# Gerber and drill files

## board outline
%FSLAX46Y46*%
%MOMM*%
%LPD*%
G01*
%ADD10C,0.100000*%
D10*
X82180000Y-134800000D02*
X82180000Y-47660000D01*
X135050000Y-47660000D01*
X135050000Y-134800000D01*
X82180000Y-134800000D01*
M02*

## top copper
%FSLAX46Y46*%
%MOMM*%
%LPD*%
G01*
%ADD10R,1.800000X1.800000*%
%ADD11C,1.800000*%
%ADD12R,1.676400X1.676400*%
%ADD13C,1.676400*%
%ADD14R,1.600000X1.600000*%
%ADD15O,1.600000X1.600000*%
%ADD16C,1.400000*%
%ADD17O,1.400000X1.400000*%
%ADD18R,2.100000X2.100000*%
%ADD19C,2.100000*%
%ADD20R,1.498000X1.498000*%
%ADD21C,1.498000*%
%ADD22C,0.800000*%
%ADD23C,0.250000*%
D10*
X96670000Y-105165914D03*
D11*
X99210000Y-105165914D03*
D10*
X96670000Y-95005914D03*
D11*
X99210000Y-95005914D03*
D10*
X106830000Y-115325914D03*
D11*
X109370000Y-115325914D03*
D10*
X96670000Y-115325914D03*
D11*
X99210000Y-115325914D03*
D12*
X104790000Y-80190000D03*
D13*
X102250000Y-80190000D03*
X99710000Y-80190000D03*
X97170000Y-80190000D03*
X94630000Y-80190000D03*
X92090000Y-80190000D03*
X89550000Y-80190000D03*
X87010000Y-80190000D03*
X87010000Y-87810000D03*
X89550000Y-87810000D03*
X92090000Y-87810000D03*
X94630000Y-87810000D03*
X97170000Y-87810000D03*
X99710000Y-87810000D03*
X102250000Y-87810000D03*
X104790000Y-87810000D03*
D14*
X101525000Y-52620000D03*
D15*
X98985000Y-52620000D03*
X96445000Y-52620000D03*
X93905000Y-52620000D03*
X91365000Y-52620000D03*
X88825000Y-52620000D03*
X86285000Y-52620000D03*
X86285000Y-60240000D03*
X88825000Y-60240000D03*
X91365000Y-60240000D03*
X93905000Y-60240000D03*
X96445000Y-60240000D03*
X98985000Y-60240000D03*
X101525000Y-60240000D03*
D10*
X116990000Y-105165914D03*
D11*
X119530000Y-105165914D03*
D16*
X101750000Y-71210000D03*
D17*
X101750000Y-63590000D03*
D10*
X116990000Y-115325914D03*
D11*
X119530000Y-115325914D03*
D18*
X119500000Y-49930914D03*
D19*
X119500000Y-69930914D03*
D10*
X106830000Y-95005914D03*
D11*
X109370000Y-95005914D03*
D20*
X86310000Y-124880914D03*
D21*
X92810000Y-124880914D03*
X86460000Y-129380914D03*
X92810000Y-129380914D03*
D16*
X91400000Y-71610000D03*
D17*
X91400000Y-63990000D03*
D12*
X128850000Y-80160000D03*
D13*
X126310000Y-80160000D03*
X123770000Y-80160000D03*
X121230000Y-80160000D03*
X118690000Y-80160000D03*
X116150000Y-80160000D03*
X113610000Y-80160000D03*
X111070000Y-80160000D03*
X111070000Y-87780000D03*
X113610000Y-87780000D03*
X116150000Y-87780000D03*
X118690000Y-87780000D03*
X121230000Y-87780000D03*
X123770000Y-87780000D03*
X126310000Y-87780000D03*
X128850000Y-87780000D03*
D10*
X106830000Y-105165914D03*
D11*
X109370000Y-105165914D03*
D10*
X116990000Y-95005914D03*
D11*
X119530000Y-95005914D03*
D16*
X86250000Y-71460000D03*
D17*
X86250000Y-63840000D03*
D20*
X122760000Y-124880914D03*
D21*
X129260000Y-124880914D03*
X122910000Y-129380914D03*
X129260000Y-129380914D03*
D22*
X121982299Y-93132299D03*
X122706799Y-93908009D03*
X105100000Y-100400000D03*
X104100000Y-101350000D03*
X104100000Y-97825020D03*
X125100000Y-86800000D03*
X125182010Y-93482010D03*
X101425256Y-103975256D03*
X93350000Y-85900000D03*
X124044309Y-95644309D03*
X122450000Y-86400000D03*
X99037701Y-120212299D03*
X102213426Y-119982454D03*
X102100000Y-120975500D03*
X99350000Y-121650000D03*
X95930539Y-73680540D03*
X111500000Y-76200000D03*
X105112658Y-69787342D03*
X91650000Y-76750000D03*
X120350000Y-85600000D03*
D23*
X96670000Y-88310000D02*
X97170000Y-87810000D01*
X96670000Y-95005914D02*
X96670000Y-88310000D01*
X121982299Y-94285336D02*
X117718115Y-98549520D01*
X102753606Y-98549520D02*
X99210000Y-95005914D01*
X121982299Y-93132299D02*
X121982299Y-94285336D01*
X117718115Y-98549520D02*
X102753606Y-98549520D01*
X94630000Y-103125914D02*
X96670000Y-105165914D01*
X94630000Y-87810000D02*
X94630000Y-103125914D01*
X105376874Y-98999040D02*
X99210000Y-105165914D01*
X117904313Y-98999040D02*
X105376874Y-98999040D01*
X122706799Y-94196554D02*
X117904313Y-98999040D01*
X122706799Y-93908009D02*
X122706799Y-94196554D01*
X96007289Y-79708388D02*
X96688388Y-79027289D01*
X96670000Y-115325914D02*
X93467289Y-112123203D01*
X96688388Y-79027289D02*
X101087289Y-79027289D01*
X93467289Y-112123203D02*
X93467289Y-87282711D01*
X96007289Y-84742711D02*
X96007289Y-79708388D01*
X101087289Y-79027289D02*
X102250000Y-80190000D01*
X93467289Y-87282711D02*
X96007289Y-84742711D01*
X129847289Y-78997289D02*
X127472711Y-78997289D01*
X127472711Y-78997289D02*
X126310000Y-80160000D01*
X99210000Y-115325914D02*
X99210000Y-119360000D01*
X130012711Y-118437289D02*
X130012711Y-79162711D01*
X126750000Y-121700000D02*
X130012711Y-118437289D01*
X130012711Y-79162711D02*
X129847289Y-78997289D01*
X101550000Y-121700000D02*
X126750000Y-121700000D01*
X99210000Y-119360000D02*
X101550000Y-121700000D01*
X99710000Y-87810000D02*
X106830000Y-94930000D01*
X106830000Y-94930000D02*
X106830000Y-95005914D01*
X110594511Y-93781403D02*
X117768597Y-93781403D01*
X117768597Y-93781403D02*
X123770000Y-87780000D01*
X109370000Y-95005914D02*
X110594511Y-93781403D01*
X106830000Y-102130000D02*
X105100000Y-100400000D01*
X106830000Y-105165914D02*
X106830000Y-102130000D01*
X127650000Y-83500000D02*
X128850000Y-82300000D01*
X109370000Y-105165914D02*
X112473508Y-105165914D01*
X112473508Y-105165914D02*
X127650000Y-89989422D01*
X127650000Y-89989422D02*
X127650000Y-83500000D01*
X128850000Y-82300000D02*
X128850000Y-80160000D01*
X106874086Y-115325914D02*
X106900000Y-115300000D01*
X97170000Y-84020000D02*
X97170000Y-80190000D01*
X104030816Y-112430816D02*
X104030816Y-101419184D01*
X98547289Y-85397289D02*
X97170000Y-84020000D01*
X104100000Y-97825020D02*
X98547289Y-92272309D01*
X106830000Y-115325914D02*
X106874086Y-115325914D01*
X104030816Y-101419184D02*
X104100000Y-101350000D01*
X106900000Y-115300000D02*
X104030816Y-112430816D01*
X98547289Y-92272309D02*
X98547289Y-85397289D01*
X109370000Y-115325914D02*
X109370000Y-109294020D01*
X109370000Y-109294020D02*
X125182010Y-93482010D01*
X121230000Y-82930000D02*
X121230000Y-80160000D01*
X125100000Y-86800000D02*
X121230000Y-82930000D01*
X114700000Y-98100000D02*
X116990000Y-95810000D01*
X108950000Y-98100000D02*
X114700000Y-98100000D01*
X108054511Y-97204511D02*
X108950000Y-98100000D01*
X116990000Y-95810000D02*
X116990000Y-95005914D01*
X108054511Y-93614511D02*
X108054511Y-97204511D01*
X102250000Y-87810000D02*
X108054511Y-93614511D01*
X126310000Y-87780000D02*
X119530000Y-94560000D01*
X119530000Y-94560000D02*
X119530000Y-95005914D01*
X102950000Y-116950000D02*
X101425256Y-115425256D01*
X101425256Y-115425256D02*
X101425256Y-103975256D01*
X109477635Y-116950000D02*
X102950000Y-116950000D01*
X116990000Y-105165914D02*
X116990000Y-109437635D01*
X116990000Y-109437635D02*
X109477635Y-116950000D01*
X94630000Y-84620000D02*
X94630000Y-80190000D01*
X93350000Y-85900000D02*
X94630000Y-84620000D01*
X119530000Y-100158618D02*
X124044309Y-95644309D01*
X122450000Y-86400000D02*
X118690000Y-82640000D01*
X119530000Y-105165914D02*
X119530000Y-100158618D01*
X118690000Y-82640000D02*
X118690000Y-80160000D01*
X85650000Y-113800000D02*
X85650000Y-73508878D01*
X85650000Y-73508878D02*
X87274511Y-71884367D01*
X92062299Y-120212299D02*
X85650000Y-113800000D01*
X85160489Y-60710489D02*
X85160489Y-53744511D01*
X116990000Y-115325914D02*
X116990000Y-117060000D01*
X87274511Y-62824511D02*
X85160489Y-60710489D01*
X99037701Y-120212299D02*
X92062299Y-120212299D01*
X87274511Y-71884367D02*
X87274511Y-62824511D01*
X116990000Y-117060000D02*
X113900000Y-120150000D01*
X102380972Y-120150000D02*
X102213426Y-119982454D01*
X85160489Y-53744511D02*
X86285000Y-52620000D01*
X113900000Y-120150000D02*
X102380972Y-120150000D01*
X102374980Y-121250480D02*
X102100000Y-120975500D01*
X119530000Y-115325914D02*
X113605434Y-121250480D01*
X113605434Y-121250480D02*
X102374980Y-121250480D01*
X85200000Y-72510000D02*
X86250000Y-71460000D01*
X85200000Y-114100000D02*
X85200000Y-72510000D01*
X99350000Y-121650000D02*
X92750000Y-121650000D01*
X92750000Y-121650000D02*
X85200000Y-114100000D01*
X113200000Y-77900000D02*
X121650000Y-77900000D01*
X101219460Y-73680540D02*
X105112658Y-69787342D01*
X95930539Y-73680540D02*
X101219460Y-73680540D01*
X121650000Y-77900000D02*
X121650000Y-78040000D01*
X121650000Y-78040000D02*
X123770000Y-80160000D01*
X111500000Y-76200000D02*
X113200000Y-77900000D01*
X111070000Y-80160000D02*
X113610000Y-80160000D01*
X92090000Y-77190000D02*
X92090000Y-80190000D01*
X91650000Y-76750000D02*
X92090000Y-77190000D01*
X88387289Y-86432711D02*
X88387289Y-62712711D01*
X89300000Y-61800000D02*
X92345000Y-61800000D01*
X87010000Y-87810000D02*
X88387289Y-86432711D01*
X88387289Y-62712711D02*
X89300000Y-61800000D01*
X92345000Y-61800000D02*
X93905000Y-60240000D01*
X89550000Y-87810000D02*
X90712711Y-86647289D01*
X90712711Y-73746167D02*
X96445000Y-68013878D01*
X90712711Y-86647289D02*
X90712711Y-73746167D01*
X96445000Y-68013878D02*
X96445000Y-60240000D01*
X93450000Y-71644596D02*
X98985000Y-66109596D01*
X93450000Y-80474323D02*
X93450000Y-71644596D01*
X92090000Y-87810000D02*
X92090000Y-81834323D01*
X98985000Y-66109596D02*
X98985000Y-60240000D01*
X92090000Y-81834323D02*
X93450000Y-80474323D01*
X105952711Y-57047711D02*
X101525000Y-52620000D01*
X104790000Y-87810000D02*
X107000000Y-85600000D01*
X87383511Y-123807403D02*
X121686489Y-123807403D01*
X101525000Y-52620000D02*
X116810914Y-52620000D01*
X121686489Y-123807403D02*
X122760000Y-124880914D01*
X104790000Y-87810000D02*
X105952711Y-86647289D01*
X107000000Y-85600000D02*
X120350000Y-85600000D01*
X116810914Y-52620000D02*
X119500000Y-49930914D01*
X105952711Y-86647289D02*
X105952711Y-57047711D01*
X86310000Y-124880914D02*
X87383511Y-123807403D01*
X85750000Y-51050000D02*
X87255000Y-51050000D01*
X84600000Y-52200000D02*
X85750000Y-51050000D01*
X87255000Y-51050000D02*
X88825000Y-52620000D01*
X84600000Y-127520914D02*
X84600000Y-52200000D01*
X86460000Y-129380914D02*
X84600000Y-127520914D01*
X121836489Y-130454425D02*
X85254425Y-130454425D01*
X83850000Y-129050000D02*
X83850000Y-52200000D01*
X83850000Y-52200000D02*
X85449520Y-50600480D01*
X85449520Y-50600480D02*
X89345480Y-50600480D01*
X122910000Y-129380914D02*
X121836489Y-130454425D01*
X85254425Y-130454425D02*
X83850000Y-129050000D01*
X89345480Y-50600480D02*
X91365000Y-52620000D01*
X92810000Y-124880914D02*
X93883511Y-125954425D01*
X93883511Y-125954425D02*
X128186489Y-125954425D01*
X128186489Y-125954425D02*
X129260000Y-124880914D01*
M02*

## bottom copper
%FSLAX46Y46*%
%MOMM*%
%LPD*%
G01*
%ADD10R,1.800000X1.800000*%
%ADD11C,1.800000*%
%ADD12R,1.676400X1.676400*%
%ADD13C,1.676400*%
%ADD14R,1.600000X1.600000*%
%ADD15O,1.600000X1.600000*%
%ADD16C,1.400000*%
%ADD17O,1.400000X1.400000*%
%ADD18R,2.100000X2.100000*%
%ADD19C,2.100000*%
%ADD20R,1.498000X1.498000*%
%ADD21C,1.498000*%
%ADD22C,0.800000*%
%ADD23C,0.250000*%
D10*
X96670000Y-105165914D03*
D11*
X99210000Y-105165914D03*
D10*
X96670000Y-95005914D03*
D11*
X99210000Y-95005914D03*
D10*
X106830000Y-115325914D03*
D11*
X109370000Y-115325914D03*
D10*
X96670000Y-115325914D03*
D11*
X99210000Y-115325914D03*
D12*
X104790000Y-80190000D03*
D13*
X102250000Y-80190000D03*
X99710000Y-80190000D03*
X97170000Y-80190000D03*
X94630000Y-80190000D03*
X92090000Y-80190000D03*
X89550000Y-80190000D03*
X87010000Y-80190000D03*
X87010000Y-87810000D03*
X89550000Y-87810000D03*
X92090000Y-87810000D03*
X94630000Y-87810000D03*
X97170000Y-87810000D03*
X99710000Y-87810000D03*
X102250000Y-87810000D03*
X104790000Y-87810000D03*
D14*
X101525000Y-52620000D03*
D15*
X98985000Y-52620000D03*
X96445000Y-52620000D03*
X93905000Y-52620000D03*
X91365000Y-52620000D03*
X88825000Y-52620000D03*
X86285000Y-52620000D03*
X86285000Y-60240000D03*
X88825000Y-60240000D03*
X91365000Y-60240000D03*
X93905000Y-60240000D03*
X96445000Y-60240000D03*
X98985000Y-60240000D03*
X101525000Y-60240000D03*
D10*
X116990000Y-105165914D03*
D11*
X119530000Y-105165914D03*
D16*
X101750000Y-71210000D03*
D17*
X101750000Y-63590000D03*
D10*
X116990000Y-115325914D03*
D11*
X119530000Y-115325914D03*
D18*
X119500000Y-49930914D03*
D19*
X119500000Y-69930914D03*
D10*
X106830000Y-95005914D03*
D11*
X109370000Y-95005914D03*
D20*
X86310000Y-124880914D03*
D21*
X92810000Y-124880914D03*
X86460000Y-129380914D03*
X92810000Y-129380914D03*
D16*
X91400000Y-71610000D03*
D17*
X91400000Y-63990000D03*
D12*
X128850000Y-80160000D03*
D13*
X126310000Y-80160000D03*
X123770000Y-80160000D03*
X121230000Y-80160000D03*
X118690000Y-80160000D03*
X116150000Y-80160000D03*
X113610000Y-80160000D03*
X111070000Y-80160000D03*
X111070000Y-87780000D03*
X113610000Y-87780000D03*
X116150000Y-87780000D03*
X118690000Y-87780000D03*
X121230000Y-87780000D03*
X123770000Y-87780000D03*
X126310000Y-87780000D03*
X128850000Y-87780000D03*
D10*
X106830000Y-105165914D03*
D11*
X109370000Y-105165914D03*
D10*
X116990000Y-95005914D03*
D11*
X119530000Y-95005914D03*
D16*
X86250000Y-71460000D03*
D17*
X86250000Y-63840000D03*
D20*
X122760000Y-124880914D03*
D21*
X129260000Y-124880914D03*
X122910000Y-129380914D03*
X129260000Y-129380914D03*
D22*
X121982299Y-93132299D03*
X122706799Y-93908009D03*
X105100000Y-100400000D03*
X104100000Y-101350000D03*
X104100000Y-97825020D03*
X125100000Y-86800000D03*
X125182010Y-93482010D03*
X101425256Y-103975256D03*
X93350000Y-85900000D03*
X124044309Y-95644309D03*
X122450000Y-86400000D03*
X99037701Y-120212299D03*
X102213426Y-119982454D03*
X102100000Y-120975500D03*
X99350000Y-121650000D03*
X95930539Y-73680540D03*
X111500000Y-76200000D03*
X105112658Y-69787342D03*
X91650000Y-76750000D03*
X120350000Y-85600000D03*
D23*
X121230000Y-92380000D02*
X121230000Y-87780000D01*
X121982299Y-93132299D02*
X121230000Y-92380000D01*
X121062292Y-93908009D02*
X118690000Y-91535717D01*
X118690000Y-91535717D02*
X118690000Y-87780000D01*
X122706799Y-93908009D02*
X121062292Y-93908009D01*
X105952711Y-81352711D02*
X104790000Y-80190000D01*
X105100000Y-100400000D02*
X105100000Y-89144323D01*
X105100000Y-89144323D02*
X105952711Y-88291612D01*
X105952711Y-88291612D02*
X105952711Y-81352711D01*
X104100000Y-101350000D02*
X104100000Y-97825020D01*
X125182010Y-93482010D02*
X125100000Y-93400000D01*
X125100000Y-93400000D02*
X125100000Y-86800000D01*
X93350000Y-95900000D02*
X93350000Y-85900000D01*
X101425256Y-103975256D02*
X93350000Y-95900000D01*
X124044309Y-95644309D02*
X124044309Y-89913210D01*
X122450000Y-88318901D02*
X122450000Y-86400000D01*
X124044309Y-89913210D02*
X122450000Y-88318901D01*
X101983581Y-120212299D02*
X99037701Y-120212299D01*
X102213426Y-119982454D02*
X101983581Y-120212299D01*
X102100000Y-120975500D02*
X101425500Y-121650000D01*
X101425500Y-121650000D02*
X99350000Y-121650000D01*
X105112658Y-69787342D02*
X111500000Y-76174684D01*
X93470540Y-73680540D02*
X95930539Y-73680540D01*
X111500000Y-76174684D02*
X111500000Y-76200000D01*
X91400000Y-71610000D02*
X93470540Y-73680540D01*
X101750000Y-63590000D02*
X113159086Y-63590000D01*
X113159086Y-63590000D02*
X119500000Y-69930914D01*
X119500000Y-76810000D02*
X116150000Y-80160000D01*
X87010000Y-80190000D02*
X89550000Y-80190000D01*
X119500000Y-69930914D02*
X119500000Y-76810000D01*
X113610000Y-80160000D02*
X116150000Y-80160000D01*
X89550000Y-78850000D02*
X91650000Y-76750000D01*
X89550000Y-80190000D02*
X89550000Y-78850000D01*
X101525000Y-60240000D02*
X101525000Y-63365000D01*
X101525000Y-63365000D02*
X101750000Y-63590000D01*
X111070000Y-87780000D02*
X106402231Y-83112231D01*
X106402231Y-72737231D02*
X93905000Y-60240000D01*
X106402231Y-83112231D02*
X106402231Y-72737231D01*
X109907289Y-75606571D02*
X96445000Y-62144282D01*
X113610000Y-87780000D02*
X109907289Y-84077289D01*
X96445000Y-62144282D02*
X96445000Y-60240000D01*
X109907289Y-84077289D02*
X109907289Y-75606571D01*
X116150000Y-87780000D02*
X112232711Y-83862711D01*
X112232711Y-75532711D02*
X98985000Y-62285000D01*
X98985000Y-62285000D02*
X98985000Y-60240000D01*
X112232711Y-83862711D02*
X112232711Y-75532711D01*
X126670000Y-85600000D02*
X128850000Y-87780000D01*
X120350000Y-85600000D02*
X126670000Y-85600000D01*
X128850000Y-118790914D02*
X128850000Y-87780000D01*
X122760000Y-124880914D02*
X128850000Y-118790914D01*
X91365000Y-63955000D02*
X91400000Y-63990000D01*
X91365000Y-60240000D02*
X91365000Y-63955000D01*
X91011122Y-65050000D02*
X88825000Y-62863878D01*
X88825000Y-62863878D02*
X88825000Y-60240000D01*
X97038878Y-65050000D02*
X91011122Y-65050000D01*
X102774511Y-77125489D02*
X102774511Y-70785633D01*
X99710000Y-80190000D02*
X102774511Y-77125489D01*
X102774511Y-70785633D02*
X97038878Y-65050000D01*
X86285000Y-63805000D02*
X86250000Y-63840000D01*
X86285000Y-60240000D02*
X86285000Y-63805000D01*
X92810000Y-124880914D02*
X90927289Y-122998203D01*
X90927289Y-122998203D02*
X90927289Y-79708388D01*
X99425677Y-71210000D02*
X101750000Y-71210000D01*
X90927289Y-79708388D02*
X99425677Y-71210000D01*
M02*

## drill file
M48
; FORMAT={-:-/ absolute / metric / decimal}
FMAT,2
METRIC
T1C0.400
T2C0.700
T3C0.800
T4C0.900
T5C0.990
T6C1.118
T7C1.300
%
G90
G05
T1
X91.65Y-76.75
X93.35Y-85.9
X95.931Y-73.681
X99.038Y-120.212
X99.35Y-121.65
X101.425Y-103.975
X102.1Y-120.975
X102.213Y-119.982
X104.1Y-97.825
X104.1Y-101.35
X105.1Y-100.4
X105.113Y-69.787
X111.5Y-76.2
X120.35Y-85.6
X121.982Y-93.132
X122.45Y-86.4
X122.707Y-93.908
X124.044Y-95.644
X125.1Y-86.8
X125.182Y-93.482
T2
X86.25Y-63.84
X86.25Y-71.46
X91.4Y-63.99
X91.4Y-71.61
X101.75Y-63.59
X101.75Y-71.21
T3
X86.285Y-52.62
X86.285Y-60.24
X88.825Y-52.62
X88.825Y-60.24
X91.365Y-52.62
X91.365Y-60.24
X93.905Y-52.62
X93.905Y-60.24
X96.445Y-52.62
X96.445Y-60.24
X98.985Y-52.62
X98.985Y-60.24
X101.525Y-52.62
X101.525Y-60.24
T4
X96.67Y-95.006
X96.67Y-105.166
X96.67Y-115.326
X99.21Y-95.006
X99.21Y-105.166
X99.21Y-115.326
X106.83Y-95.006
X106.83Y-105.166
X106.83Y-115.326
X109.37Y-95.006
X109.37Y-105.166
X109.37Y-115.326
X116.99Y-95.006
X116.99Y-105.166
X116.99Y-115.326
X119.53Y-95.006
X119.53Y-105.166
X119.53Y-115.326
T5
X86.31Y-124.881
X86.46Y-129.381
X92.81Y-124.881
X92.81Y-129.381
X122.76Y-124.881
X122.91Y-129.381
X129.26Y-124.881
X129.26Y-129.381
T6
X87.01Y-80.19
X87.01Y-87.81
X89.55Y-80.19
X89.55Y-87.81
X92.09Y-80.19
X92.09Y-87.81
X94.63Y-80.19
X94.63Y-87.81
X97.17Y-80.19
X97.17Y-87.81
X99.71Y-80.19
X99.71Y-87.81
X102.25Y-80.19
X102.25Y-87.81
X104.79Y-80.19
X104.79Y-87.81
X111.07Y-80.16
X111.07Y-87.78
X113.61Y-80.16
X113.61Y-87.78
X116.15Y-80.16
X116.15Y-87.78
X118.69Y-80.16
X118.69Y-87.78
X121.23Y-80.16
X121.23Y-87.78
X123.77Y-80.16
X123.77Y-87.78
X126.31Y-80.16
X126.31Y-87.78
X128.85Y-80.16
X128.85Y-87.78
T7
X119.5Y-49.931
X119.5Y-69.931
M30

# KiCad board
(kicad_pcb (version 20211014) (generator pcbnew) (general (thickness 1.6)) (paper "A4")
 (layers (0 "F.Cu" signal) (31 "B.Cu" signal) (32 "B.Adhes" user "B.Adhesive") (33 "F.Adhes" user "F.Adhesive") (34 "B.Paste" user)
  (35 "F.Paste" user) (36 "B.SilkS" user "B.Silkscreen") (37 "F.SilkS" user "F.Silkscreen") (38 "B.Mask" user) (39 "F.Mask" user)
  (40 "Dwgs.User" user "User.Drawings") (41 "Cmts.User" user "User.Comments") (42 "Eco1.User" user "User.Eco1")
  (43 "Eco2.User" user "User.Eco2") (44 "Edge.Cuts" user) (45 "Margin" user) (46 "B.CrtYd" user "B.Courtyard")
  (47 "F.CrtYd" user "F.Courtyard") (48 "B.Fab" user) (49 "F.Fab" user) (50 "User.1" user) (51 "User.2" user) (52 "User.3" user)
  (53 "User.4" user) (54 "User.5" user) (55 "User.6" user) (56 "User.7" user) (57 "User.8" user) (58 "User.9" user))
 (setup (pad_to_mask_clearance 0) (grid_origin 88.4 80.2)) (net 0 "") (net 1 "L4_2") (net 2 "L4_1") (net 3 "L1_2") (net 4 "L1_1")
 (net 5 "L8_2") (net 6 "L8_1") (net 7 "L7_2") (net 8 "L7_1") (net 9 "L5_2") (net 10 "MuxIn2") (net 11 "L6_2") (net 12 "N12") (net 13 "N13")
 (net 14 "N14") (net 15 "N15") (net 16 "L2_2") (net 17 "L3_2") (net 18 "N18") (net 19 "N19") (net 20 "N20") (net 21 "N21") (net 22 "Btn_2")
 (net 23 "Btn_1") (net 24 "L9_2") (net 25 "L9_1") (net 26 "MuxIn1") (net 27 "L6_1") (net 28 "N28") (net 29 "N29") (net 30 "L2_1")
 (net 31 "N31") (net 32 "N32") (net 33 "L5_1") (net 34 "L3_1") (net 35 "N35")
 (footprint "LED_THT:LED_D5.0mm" (layer "F.Cu") (at 96.67 105.165914)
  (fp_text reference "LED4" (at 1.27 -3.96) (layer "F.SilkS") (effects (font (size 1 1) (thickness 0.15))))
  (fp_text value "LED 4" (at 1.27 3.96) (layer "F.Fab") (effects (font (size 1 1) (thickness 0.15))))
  (pad "1" thru_hole rect (at 0 0) (size 1.8 1.8) (drill 0.9) (layers *.Cu *.Mask) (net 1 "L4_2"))
  (pad "2" thru_hole circle (at 2.54 0) (size 1.8 1.8) (drill 0.9) (layers *.Cu *.Mask) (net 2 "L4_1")))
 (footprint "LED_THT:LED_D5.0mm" (layer "F.Cu") (at 96.67 95.005914)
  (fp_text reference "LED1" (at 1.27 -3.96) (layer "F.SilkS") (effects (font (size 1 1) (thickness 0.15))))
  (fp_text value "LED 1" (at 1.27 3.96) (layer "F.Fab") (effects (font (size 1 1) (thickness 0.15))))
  (pad "1" thru_hole rect (at 0 0) (size 1.8 1.8) (drill 0.9) (layers *.Cu *.Mask) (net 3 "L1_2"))
  (pad "2" thru_hole circle (at 2.54 0) (size 1.8 1.8) (drill 0.9) (layers *.Cu *.Mask) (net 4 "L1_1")))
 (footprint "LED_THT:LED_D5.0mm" (layer "F.Cu") (at 106.83 115.325914)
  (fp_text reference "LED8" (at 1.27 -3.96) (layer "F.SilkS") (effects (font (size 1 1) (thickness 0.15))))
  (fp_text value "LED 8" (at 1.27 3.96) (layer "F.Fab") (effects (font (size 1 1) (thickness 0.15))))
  (pad "1" thru_hole rect (at 0 0) (size 1.8 1.8) (drill 0.9) (layers *.Cu *.Mask) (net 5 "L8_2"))
  (pad "2" thru_hole circle (at 2.54 0) (size 1.8 1.8) (drill 0.9) (layers *.Cu *.Mask) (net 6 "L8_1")))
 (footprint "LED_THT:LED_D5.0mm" (layer "F.Cu") (at 96.67 115.325914)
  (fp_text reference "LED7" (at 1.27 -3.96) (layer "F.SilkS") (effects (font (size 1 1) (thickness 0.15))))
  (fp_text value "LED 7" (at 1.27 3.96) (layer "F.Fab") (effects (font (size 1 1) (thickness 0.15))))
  (pad "1" thru_hole rect (at 0 0) (size 1.8 1.8) (drill 0.9) (layers *.Cu *.Mask) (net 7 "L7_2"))
  (pad "2" thru_hole circle (at 2.54 0) (size 1.8 1.8) (drill 0.9) (layers *.Cu *.Mask) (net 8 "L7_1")))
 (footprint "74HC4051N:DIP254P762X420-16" (layer "F.Cu") (at 87.01 87.81 -90)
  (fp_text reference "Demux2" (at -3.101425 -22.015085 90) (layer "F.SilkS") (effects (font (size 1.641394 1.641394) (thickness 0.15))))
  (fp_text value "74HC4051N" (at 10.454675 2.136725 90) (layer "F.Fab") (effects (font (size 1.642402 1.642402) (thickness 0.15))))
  (pad "1" thru_hole rect locked (at -7.62 -17.78 270) (size 1.6764 1.6764) (drill 1.1176) (layers *.Cu *.Mask) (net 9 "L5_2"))
  (pad "2" thru_hole circle locked (at -7.62 -15.24 270) (size 1.6764 1.6764) (drill 1.1176) (layers *.Cu *.Mask) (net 7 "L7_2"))
  (pad "3" thru_hole circle locked (at -7.62 -12.7 270) (size 1.6764 1.6764) (drill 1.1176) (layers *.Cu *.Mask) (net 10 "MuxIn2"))
  (pad "4" thru_hole circle locked (at -7.62 -10.16 270) (size 1.6764 1.6764) (drill 1.1176) (layers *.Cu *.Mask) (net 5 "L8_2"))
  (pad "5" thru_hole circle locked (at -7.62 -7.62 270) (size 1.6764 1.6764) (drill 1.1176) (layers *.Cu *.Mask) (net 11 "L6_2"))
  (pad "6" thru_hole circle locked (at -7.62 -5.08 270) (size 1.6764 1.6764) (drill 1.1176) (layers *.Cu *.Mask) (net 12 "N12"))
  (pad "7" thru_hole circle locked (at -7.62 -2.54 270) (size 1.6764 1.6764) (drill 1.1176) (layers *.Cu *.Mask) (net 12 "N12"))
  (pad "8" thru_hole circle locked (at -7.62 0 270) (size 1.6764 1.6764) (drill 1.1176) (layers *.Cu *.Mask) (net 12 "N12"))
  (pad "9" thru_hole circle locked (at 0 0 270) (size 1.6764 1.6764) (drill 1.1176) (layers *.Cu *.Mask) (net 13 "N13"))
  (pad "10" thru_hole circle locked (at 0 -2.54 270) (size 1.6764 1.6764) (drill 1.1176) (layers *.Cu *.Mask) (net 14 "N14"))
  (pad "11" thru_hole circle locked (at 0 -5.08 270) (size 1.6764 1.6764) (drill 1.1176) (layers *.Cu *.Mask) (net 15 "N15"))
  (pad "12" thru_hole circle locked (at 0 -7.62 270) (size 1.6764 1.6764) (drill 1.1176) (layers *.Cu *.Mask) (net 1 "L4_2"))
  (pad "13" thru_hole circle locked (at 0 -10.16 270) (size 1.6764 1.6764) (drill 1.1176) (layers *.Cu *.Mask) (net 3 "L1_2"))
  (pad "14" thru_hole circle locked (at 0 -12.7 270) (size 1.6764 1.6764) (drill 1.1176) (layers *.Cu *.Mask) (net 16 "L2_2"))
  (pad "15" thru_hole circle locked (at 0 -15.24 270) (size 1.6764 1.6764) (drill 1.1176) (layers *.Cu *.Mask) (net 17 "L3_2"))
  (pad "16" thru_hole circle locked (at 0 -17.78 270) (size 1.6764 1.6764) (drill 1.1176) (layers *.Cu *.Mask) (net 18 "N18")))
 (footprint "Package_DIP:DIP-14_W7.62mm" (layer "F.Cu") (at 101.525 52.62 -90)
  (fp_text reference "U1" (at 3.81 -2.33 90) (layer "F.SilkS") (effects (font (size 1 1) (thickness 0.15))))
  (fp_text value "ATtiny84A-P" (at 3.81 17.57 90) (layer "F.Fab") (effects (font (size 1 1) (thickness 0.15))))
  (pad "1" thru_hole rect (at 0 0 270) (size 1.6 1.6) (drill 0.8) (layers *.Cu *.Mask) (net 18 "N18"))
  (pad "2" thru_hole oval (at 0 2.54 270) (size 1.6 1.6) (drill 0.8) (layers *.Cu *.Mask) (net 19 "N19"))
  (pad "3" thru_hole oval (at 0 5.08 270) (size 1.6 1.6) (drill 0.8) (layers *.Cu *.Mask) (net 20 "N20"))
  (pad "4" thru_hole oval (at 0 7.62 270) (size 1.6 1.6) (drill 0.8) (layers *.Cu *.Mask) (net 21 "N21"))
  (pad "5" thru_hole oval (at 0 10.16 270) (size 1.6 1.6) (drill 0.8) (layers *.Cu *.Mask) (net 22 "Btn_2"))
  (pad "6" thru_hole oval (at 0 12.7 270) (size 1.6 1.6) (drill 0.8) (layers *.Cu *.Mask) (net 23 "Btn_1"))
  (pad "7" thru_hole oval (at 0 15.24 270) (size 1.6 1.6) (drill 0.8) (layers *.Cu *.Mask) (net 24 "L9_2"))
  (pad "8" thru_hole oval (at 7.62 15.24 270) (size 1.6 1.6) (drill 0.8) (layers *.Cu *.Mask) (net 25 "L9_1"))
  (pad "9" thru_hole oval (at 7.62 12.7 270) (size 1.6 1.6) (drill 0.8) (layers *.Cu *.Mask) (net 10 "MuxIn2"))
  (pad "10" thru_hole oval (at 7.62 10.16 270) (size 1.6 1.6) (drill 0.8) (layers *.Cu *.Mask) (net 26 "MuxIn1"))
  (pad "11" thru_hole oval (at 7.62 7.62 270) (size 1.6 1.6) (drill 0.8) (layers *.Cu *.Mask) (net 13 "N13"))
  (pad "12" thru_hole oval (at 7.62 5.08 270) (size 1.6 1.6) (drill 0.8) (layers *.Cu *.Mask) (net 14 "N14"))
  (pad "13" thru_hole oval (at 7.62 2.54 270) (size 1.6 1.6) (drill 0.8) (layers *.Cu *.Mask) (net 15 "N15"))
  (pad "14" thru_hole oval (at 7.62 0 270) (size 1.6 1.6) (drill 0.8) (layers *.Cu *.Mask) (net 12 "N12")))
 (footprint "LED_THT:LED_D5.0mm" (layer "F.Cu") (at 116.99 105.165914)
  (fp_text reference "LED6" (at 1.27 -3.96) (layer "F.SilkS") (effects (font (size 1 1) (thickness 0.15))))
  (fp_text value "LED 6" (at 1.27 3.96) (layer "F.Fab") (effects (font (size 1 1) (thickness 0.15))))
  (pad "1" thru_hole rect (at 0 0) (size 1.8 1.8) (drill 0.9) (layers *.Cu *.Mask) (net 11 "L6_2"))
  (pad "2" thru_hole circle (at 2.54 0) (size 1.8 1.8) (drill 0.9) (layers *.Cu *.Mask) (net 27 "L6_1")))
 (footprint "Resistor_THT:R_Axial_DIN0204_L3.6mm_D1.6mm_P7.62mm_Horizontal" (layer "F.Cu") (at 101.75 71.21 90)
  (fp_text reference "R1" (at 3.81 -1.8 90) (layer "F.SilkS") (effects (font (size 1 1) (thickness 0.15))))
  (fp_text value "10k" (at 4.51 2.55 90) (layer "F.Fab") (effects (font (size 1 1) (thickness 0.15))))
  (pad "1" thru_hole circle (at 0 0 90) (size 1.4 1.4) (drill 0.7) (layers *.Cu *.Mask) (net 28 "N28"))
  (pad "2" thru_hole oval (at 7.62 0 90) (size 1.4 1.4) (drill 0.7) (layers *.Cu *.Mask) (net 12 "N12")))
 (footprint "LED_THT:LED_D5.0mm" (layer "F.Cu") (at 116.99 115.325914)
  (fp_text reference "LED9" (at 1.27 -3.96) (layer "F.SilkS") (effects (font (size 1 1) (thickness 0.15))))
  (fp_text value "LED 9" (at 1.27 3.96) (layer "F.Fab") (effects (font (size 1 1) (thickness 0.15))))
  (pad "1" thru_hole rect (at 0 0) (size 1.8 1.8) (drill 0.9) (layers *.Cu *.Mask) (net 24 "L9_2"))
  (pad "2" thru_hole circle (at 2.54 0) (size 1.8 1.8) (drill 0.9) (layers *.Cu *.Mask) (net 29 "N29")))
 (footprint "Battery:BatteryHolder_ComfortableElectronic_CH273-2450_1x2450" (layer "F.Cu") (at 119.5 49.930914 -90)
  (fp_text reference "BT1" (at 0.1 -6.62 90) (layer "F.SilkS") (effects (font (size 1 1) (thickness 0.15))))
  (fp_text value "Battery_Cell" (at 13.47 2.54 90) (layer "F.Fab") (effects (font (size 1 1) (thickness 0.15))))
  (pad "1" thru_hole rect (at 0 0 180) (size 2.1 2.1) (drill 1.3) (layers *.Cu *.Mask) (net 18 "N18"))
  (pad "2" thru_hole circle (at 20 0 180) (size 2.1 2.1) (drill 1.3) (layers *.Cu *.Mask) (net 12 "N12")))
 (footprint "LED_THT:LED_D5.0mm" (layer "F.Cu") (at 106.83 95.005914)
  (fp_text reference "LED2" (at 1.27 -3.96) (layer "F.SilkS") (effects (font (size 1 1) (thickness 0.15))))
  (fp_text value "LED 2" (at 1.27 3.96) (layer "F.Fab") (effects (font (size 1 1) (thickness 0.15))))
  (pad "1" thru_hole rect (at 0 0) (size 1.8 1.8) (drill 0.9) (layers *.Cu *.Mask) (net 16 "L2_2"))
  (pad "2" thru_hole circle (at 2.54 0) (size 1.8 1.8) (drill 0.9) (layers *.Cu *.Mask) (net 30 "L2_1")))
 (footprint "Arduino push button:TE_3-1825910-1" (layer "F.Cu") (at 89.56 127.130914)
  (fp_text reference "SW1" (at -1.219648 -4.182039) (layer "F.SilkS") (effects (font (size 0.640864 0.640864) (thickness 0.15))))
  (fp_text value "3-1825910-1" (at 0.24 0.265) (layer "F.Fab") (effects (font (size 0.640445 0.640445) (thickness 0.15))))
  (pad "1" thru_hole rect locked (at -3.25 -2.25) (size 1.498 1.498) (drill 0.99) (layers *.Cu *.Mask) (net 18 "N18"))
  (pad "2" thru_hole circle locked (at 3.25 -2.25) (size 1.498 1.498) (drill 0.99) (layers *.Cu *.Mask) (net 28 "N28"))
  (pad "3" thru_hole circle locked (at -3.1 2.25) (size 1.498 1.498) (drill 0.99) (layers *.Cu *.Mask) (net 23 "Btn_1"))
  (pad "4" thru_hole circle locked (at 3.25 2.25) (size 1.498 1.498) (drill 0.99) (layers *.Cu *.Mask) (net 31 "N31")))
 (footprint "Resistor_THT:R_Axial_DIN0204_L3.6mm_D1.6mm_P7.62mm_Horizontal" (layer "F.Cu") (at 91.4 71.61 90)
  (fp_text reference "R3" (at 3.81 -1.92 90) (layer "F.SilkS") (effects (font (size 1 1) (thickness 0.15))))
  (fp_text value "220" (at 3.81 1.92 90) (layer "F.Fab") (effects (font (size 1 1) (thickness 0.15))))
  (pad "1" thru_hole circle (at 0 0 90) (size 1.4 1.4) (drill 0.7) (layers *.Cu *.Mask) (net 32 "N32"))
  (pad "2" thru_hole oval (at 7.62 0 90) (size 1.4 1.4) (drill 0.7) (layers *.Cu *.Mask) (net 26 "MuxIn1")))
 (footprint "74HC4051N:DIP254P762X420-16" (layer "F.Cu") (at 111.07 87.78 -90)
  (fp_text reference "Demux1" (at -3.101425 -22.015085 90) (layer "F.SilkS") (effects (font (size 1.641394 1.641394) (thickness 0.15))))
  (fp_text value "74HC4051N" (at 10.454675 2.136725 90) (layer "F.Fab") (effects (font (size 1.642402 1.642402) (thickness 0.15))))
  (pad "1" thru_hole rect locked (at -7.62 -17.78 270) (size 1.6764 1.6764) (drill 1.1176) (layers *.Cu *.Mask) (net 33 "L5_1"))
  (pad "2" thru_hole circle locked (at -7.62 -15.24 270) (size 1.6764 1.6764) (drill 1.1176) (layers *.Cu *.Mask) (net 8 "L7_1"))
  (pad "3" thru_hole circle locked (at -7.62 -12.7 270) (size 1.6764 1.6764) (drill 1.1176) (layers *.Cu *.Mask) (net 32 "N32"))
  (pad "4" thru_hole circle locked (at -7.62 -10.16 270) (size 1.6764 1.6764) (drill 1.1176) (layers *.Cu *.Mask) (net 6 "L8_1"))
  (pad "5" thru_hole circle locked (at -7.62 -7.62 270) (size 1.6764 1.6764) (drill 1.1176) (layers *.Cu *.Mask) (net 27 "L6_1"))
  (pad "6" thru_hole circle locked (at -7.62 -5.08 270) (size 1.6764 1.6764) (drill 1.1176) (layers *.Cu *.Mask) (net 12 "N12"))
  (pad "7" thru_hole circle locked (at -7.62 -2.54 270) (size 1.6764 1.6764) (drill 1.1176) (layers *.Cu *.Mask) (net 12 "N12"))
  (pad "8" thru_hole circle locked (at -7.62 0 270) (size 1.6764 1.6764) (drill 1.1176) (layers *.Cu *.Mask) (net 12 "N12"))
  (pad "9" thru_hole circle locked (at 0 0 270) (size 1.6764 1.6764) (drill 1.1176) (layers *.Cu *.Mask) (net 13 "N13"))
  (pad "10" thru_hole circle locked (at 0 -2.54 270) (size 1.6764 1.6764) (drill 1.1176) (layers *.Cu *.Mask) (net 14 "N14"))
  (pad "11" thru_hole circle locked (at 0 -5.08 270) (size 1.6764 1.6764) (drill 1.1176) (layers *.Cu *.Mask) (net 15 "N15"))
  (pad "12" thru_hole circle locked (at 0 -7.62 270) (size 1.6764 1.6764) (drill 1.1176) (layers *.Cu *.Mask) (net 2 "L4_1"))
  (pad "13" thru_hole circle locked (at 0 -10.16 270) (size 1.6764 1.6764) (drill 1.1176) (layers *.Cu *.Mask) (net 4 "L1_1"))
  (pad "14" thru_hole circle locked (at 0 -12.7 270) (size 1.6764 1.6764) (drill 1.1176) (layers *.Cu *.Mask) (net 30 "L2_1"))
  (pad "15" thru_hole circle locked (at 0 -15.24 270) (size 1.6764 1.6764) (drill 1.1176) (layers *.Cu *.Mask) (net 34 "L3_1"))
  (pad "16" thru_hole circle locked (at 0 -17.78 270) (size 1.6764 1.6764) (drill 1.1176) (layers *.Cu *.Mask) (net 18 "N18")))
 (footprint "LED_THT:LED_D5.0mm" (layer "F.Cu") (at 106.83 105.165914)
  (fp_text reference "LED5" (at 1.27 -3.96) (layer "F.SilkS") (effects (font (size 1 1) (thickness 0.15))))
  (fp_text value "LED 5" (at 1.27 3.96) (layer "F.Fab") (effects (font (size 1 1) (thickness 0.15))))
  (pad "1" thru_hole rect (at 0 0) (size 1.8 1.8) (drill 0.9) (layers *.Cu *.Mask) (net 9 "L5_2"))
  (pad "2" thru_hole circle (at 2.54 0) (size 1.8 1.8) (drill 0.9) (layers *.Cu *.Mask) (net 33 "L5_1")))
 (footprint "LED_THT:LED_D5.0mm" (layer "F.Cu") (at 116.99 95.005914)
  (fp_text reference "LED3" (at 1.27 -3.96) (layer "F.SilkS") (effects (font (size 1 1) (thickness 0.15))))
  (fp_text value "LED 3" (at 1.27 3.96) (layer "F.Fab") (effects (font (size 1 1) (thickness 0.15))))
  (pad "1" thru_hole rect (at 0 0) (size 1.8 1.8) (drill 0.9) (layers *.Cu *.Mask) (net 17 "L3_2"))
  (pad "2" thru_hole circle (at 2.54 0) (size 1.8 1.8) (drill 0.9) (layers *.Cu *.Mask) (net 34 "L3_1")))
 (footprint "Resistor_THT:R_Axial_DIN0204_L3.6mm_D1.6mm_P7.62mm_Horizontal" (layer "F.Cu") (at 86.25 71.46 90)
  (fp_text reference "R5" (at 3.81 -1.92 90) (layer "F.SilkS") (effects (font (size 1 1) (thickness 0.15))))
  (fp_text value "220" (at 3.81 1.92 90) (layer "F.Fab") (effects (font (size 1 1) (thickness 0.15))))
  (pad "1" thru_hole circle (at 0 0 90) (size 1.4 1.4) (drill 0.7) (layers *.Cu *.Mask) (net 29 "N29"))
  (pad "2" thru_hole oval (at 7.62 0 90) (size 1.4 1.4) (drill 0.7) (layers *.Cu *.Mask) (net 25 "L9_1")))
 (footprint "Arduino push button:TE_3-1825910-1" (layer "F.Cu") (at 126.01 127.130914)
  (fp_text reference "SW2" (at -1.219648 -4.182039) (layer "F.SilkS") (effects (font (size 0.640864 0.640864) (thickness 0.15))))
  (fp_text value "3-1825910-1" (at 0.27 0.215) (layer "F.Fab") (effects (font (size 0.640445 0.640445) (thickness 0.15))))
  (pad "1" thru_hole rect locked (at -3.25 -2.25) (size 1.498 1.498) (drill 0.99) (layers *.Cu *.Mask) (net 18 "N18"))
  (pad "2" thru_hole circle locked (at 3.25 -2.25) (size 1.498 1.498) (drill 0.99) (layers *.Cu *.Mask) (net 28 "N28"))
  (pad "3" thru_hole circle locked (at -3.1 2.25) (size 1.498 1.498) (drill 0.99) (layers *.Cu *.Mask) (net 22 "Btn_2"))
  (pad "4" thru_hole circle locked (at 3.25 2.25) (size 1.498 1.498) (drill 0.99) (layers *.Cu *.Mask) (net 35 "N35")))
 (gr_poly (pts (xy 82.18 134.8) (xy 82.18 47.66) (xy 135.05 47.66) (xy 135.05 134.8)) (layer "Edge.Cuts") (width 0.1) (fill none))
 (segment (start 96.67 88.31) (end 97.17 87.81) (width 0.25) (layer "F.Cu") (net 3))
 (segment (start 96.67 95.005914) (end 96.67 88.31) (width 0.25) (layer "F.Cu") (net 3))
 (segment (start 121.982299 94.285336) (end 117.718115 98.54952) (width 0.25) (layer "F.Cu") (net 4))
 (segment (start 102.753606 98.54952) (end 99.21 95.005914) (width 0.25) (layer "F.Cu") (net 4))
 (segment (start 121.982299 93.132299) (end 121.982299 94.285336) (width 0.25) (layer "F.Cu") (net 4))
 (segment (start 117.718115 98.54952) (end 102.753606 98.54952) (width 0.25) (layer "F.Cu") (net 4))
 (via (at 121.982299 93.132299) (size 0.8) (drill 0.4) (layers "F.Cu" "B.Cu") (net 4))
 (segment (start 121.23 92.38) (end 121.23 87.78) (width 0.25) (layer "B.Cu") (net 4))
 (segment (start 121.982299 93.132299) (end 121.23 92.38) (width 0.25) (layer "B.Cu") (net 4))
 (segment (start 94.63 103.125914) (end 96.67 105.165914) (width 0.25) (layer "F.Cu") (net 1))
 (segment (start 94.63 87.81) (end 94.63 103.125914) (width 0.25) (layer "F.Cu") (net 1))
 (segment (start 105.376874 98.99904) (end 99.21 105.165914) (width 0.25) (layer "F.Cu") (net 2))
 (segment (start 117.904313 98.99904) (end 105.376874 98.99904) (width 0.25) (layer "F.Cu") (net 2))
 (segment (start 122.706799 94.196554) (end 117.904313 98.99904) (width 0.25) (layer "F.Cu") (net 2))
 (segment (start 122.706799 93.908009) (end 122.706799 94.196554) (width 0.25) (layer "F.Cu") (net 2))
 (via (at 122.706799 93.908009) (size 0.8) (drill 0.4) (layers "F.Cu" "B.Cu") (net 2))
 (segment (start 121.062292 93.908009) (end 118.69 91.535717) (width 0.25) (layer "B.Cu") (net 2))
 (segment (start 118.69 91.535717) (end 118.69 87.78) (width 0.25) (layer "B.Cu") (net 2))
 (segment (start 122.706799 93.908009) (end 121.062292 93.908009) (width 0.25) (layer "B.Cu") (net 2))
 (segment (start 96.007289 79.708388) (end 96.688388 79.027289) (width 0.25) (layer "F.Cu") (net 7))
 (segment (start 96.67 115.325914) (end 93.467289 112.123203) (width 0.25) (layer "F.Cu") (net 7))
 (segment (start 96.688388 79.027289) (end 101.087289 79.027289) (width 0.25) (layer "F.Cu") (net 7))
 (segment (start 93.467289 112.123203) (end 93.467289 87.282711) (width 0.25) (layer "F.Cu") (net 7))
 (segment (start 96.007289 84.742711) (end 96.007289 79.708388) (width 0.25) (layer "F.Cu") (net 7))
 (segment (start 101.087289 79.027289) (end 102.25 80.19) (width 0.25) (layer "F.Cu") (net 7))
 (segment (start 93.467289 87.282711) (end 96.007289 84.742711) (width 0.25) (layer "F.Cu") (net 7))
 (segment (start 129.847289 78.997289) (end 127.472711 78.997289) (width 0.25) (layer "F.Cu") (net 8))
 (segment (start 127.472711 78.997289) (end 126.31 80.16) (width 0.25) (layer "F.Cu") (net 8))
 (segment (start 99.21 115.325914) (end 99.21 119.36) (width 0.25) (layer "F.Cu") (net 8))
 (segment (start 130.012711 118.437289) (end 130.012711 79.162711) (width 0.25) (layer "F.Cu") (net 8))
 (segment (start 126.75 121.7) (end 130.012711 118.437289) (width 0.25) (layer "F.Cu") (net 8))
 (segment (start 130.012711 79.162711) (end 129.847289 78.997289) (width 0.25) (layer "F.Cu") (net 8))
 (segment (start 101.55 121.7) (end 126.75 121.7) (width 0.25) (layer "F.Cu") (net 8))
 (segment (start 99.21 119.36) (end 101.55 121.7) (width 0.25) (layer "F.Cu") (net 8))
 (segment (start 99.71 87.81) (end 106.83 94.93) (width 0.25) (layer "F.Cu") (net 16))
 (segment (start 106.83 94.93) (end 106.83 95.005914) (width 0.25) (layer "F.Cu") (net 16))
 (segment (start 110.594511 93.781403) (end 117.768597 93.781403) (width 0.25) (layer "F.Cu") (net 30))
 (segment (start 117.768597 93.781403) (end 123.77 87.78) (width 0.25) (layer "F.Cu") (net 30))
 (segment (start 109.37 95.005914) (end 110.594511 93.781403) (width 0.25) (layer "F.Cu") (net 30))
 (segment (start 106.83 102.13) (end 105.1 100.4) (width 0.25) (layer "F.Cu") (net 9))
 (segment (start 106.83 105.165914) (end 106.83 102.13) (width 0.25) (layer "F.Cu") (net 9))
 (via (at 105.1 100.4) (size 0.8) (drill 0.4) (layers "F.Cu" "B.Cu") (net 9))
 (segment (start 105.952711 81.352711) (end 104.79 80.19) (width 0.25) (layer "B.Cu") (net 9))
 (segment (start 105.1 100.4) (end 105.1 89.144323) (width 0.25) (layer "B.Cu") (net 9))
 (segment (start 105.1 89.144323) (end 105.952711 88.291612) (width 0.25) (layer "B.Cu") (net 9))
 (segment (start 105.952711 88.291612) (end 105.952711 81.352711) (width 0.25) (layer "B.Cu") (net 9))
 (segment (start 127.65 83.5) (end 128.85 82.3) (width 0.25) (layer "F.Cu") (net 33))
 (segment (start 109.37 105.165914) (end 112.473508 105.165914) (width 0.25) (layer "F.Cu") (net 33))
 (segment (start 112.473508 105.165914) (end 127.65 89.989422) (width 0.25) (layer "F.Cu") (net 33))
 (segment (start 127.65 89.989422) (end 127.65 83.5) (width 0.25) (layer "F.Cu") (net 33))
 (segment (start 128.85 82.3) (end 128.85 80.16) (width 0.25) (layer "F.Cu") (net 33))
 (segment (start 106.874086 115.325914) (end 106.9 115.3) (width 0.25) (layer "F.Cu") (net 5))
 (segment (start 97.17 84.02) (end 97.17 80.19) (width 0.25) (layer "F.Cu") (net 5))
 (segment (start 104.030816 112.430816) (end 104.030816 101.419184) (width 0.25) (layer "F.Cu") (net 5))
 (segment (start 98.547289 85.397289) (end 97.17 84.02) (width 0.25) (layer "F.Cu") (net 5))
 (segment (start 104.1 97.82502) (end 98.547289 92.272309) (width 0.25) (layer "F.Cu") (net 5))
 (segment (start 106.83 115.325914) (end 106.874086 115.325914) (width 0.25) (layer "F.Cu") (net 5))
 (segment (start 104.030816 101.419184) (end 104.1 101.35) (width 0.25) (layer "F.Cu") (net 5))
 (segment (start 106.9 115.3) (end 104.030816 112.430816) (width 0.25) (layer "F.Cu") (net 5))
 (segment (start 98.547289 92.272309) (end 98.547289 85.397289) (width 0.25) (layer "F.Cu") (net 5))
 (via (at 104.1 101.35) (size 0.8) (drill 0.4) (layers "F.Cu" "B.Cu") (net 5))
 (via (at 104.1 97.82502) (size 0.8) (drill 0.4) (layers "F.Cu" "B.Cu") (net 5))
 (segment (start 104.1 101.35) (end 104.1 97.82502) (width 0.25) (layer "B.Cu") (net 5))
 (segment (start 109.37 115.325914) (end 109.37 109.29402) (width 0.25) (layer "F.Cu") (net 6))
 (segment (start 109.37 109.29402) (end 125.18201 93.48201) (width 0.25) (layer "F.Cu") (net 6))
 (segment (start 121.23 82.93) (end 121.23 80.16) (width 0.25) (layer "F.Cu") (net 6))
 (segment (start 125.1 86.8) (end 121.23 82.93) (width 0.25) (layer "F.Cu") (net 6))
 (via (at 125.1 86.8) (size 0.8) (drill 0.4) (layers "F.Cu" "B.Cu") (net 6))
 (via (at 125.18201 93.48201) (size 0.8) (drill 0.4) (layers "F.Cu" "B.Cu") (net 6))
 (segment (start 125.18201 93.48201) (end 125.1 93.4) (width 0.25) (layer "B.Cu") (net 6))
 (segment (start 125.1 93.4) (end 125.1 86.8) (width 0.25) (layer "B.Cu") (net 6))
 (segment (start 114.7 98.1) (end 116.99 95.81) (width 0.25) (layer "F.Cu") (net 17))
 (segment (start 108.95 98.1) (end 114.7 98.1) (width 0.25) (layer "F.Cu") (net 17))
 (segment (start 108.054511 97.204511) (end 108.95 98.1) (width 0.25) (layer "F.Cu") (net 17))
 (segment (start 116.99 95.81) (end 116.99 95.005914) (width 0.25) (layer "F.Cu") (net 17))
 (segment (start 108.054511 93.614511) (end 108.054511 97.204511) (width 0.25) (layer "F.Cu") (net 17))
 (segment (start 102.25 87.81) (end 108.054511 93.614511) (width 0.25) (layer "F.Cu") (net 17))
 (segment (start 126.31 87.78) (end 119.53 94.56) (width 0.25) (layer "F.Cu") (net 34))
 (segment (start 119.53 94.56) (end 119.53 95.005914) (width 0.25) (layer "F.Cu") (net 34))
 (segment (start 102.95 116.95) (end 101.425256 115.425256) (width 0.25) (layer "F.Cu") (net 11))
 (segment (start 101.425256 115.425256) (end 101.425256 103.975256) (width 0.25) (layer "F.Cu") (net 11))
 (segment (start 109.477635 116.95) (end 102.95 116.95) (width 0.25) (layer "F.Cu") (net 11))
 (segment (start 116.99 105.165914) (end 116.99 109.437635) (width 0.25) (layer "F.Cu") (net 11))
 (segment (start 116.99 109.437635) (end 109.477635 116.95) (width 0.25) (layer "F.Cu") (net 11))
 (segment (start 94.63 84.62) (end 94.63 80.19) (width 0.25) (layer "F.Cu") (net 11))
 (segment (start 93.35 85.9) (end 94.63 84.62) (width 0.25) (layer "F.Cu") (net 11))
 (via (at 101.425256 103.975256) (size 0.8) (drill 0.4) (layers "F.Cu" "B.Cu") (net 11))
 (via (at 93.35 85.9) (size 0.8) (drill 0.4) (layers "F.Cu" "B.Cu") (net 11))
 (segment (start 93.35 95.9) (end 93.35 85.9) (width 0.25) (layer "B.Cu") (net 11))
 (segment (start 101.425256 103.975256) (end 93.35 95.9) (width 0.25) (layer "B.Cu") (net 11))
 (segment (start 119.53 100.158618) (end 124.044309 95.644309) (width 0.25) (layer "F.Cu") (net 27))
 (segment (start 122.45 86.4) (end 118.69 82.64) (width 0.25) (layer "F.Cu") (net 27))
 (segment (start 119.53 105.165914) (end 119.53 100.158618) (width 0.25) (layer "F.Cu") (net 27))
 (segment (start 118.69 82.64) (end 118.69 80.16) (width 0.25) (layer "F.Cu") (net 27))
 (via (at 124.044309 95.644309) (size 0.8) (drill 0.4) (layers "F.Cu" "B.Cu") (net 27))
 (via (at 122.45 86.4) (size 0.8) (drill 0.4) (layers "F.Cu" "B.Cu") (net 27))
 (segment (start 124.044309 95.644309) (end 124.044309 89.91321) (width 0.25) (layer "B.Cu") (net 27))
 (segment (start 122.45 88.318901) (end 122.45 86.4) (width 0.25) (layer "B.Cu") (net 27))
 (segment (start 124.044309 89.91321) (end 122.45 88.318901) (width 0.25) (layer "B.Cu") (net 27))
 (segment (start 85.65 113.8) (end 85.65 73.508878) (width 0.25) (layer "F.Cu") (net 24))
 (segment (start 85.65 73.508878) (end 87.274511 71.884367) (width 0.25) (layer "F.Cu") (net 24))
 (segment (start 92.062299 120.212299) (end 85.65 113.8) (width 0.25) (layer "F.Cu") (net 24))
 (segment (start 85.160489 60.710489) (end 85.160489 53.744511) (width 0.25) (layer "F.Cu") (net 24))
 (segment (start 116.99 115.325914) (end 116.99 117.06) (width 0.25) (layer "F.Cu") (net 24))
 (segment (start 87.274511 62.824511) (end 85.160489 60.710489) (width 0.25) (layer "F.Cu") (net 24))
 (segment (start 99.037701 120.212299) (end 92.062299 120.212299) (width 0.25) (layer "F.Cu") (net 24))
 (segment (start 87.274511 71.884367) (end 87.274511 62.824511) (width 0.25) (layer "F.Cu") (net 24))
 (segment (start 116.99 117.06) (end 113.9 120.15) (width 0.25) (layer "F.Cu") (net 24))
 (segment (start 102.380972 120.15) (end 102.213426 119.982454) (width 0.25) (layer "F.Cu") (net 24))
 (segment (start 85.160489 53.744511) (end 86.285 52.62) (width 0.25) (layer "F.Cu") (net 24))
 (segment (start 113.9 120.15) (end 102.380972 120.15) (width 0.25) (layer "F.Cu") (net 24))
 (via (at 99.037701 120.212299) (size 0.8) (drill 0.4) (layers "F.Cu" "B.Cu") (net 24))
 (via (at 102.213426 119.982454) (size 0.8) (drill 0.4) (layers "F.Cu" "B.Cu") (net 24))
 (segment (start 101.983581 120.212299) (end 99.037701 120.212299) (width 0.25) (layer "B.Cu") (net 24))
 (segment (start 102.213426 119.982454) (end 101.983581 120.212299) (width 0.25) (layer "B.Cu") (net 24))
 (segment (start 102.37498 121.25048) (end 102.1 120.9755) (width 0.25) (layer "F.Cu") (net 29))
 (segment (start 119.53 115.325914) (end 113.605434 121.25048) (width 0.25) (layer "F.Cu") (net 29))
 (segment (start 113.605434 121.25048) (end 102.37498 121.25048) (width 0.25) (layer "F.Cu") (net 29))
 (segment (start 85.2 72.51) (end 86.25 71.46) (width 0.25) (layer "F.Cu") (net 29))
 (segment (start 85.2 114.1) (end 85.2 72.51) (width 0.25) (layer "F.Cu") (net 29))
 (segment (start 99.35 121.65) (end 92.75 121.65) (width 0.25) (layer "F.Cu") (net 29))
 (segment (start 92.75 121.65) (end 85.2 114.1) (width 0.25) (layer "F.Cu") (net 29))
 (via (at 102.1 120.9755) (size 0.8) (drill 0.4) (layers "F.Cu" "B.Cu") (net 29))
 (via (at 99.35 121.65) (size 0.8) (drill 0.4) (layers "F.Cu" "B.Cu") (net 29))
 (segment (start 102.1 120.9755) (end 101.4255 121.65) (width 0.25) (layer "B.Cu") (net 29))
 (segment (start 101.4255 121.65) (end 99.35 121.65) (width 0.25) (layer "B.Cu") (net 29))
 (segment (start 113.2 77.9) (end 121.65 77.9) (width 0.25) (layer "F.Cu") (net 32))
 (segment (start 101.21946 73.68054) (end 105.112658 69.787342) (width 0.25) (layer "F.Cu") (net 32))
 (segment (start 95.930539 73.68054) (end 101.21946 73.68054) (width 0.25) (layer "F.Cu") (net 32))
 (segment (start 121.65 77.9) (end 121.65 78.04) (width 0.25) (layer "F.Cu") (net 32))
 (segment (start 121.65 78.04) (end 123.77 80.16) (width 0.25) (layer "F.Cu") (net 32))
 (segment (start 111.5 76.2) (end 113.2 77.9) (width 0.25) (layer "F.Cu") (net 32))
 (via (at 95.930539 73.68054) (size 0.8) (drill 0.4) (layers "F.Cu" "B.Cu") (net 32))
 (via (at 111.5 76.2) (size 0.8) (drill 0.4) (layers "F.Cu" "B.Cu") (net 32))
 (via (at 105.112658 69.787342) (size 0.8) (drill 0.4) (layers "F.Cu" "B.Cu") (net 32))
 (segment (start 105.112658 69.787342) (end 111.5 76.174684) (width 0.25) (layer "B.Cu") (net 32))
 (segment (start 93.47054 73.68054) (end 95.930539 73.68054) (width 0.25) (layer "B.Cu") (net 32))
 (segment (start 111.5 76.174684) (end 111.5 76.2) (width 0.25) (layer "B.Cu") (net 32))
 (segment (start 91.4 71.61) (end 93.47054 73.68054) (width 0.25) (layer "B.Cu") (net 32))
 (segment (start 111.07 80.16) (end 113.61 80.16) (width 0.25) (layer "F.Cu") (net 12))
 (segment (start 92.09 77.19) (end 92.09 80.19) (width 0.25) (layer "F.Cu") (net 12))
 (segment (start 91.65 76.75) (end 92.09 77.19) (width 0.25) (layer "F.Cu") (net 12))
 (via (at 91.65 76.75) (size 0.8) (drill 0.4) (layers "F.Cu" "B.Cu") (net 12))
 (segment (start 101.75 63.59) (end 113.159086 63.59) (width 0.25) (layer "B.Cu") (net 12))
 (segment (start 113.159086 63.59) (end 119.5 69.930914) (width 0.25) (layer "B.Cu") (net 12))
 (segment (start 119.5 76.81) (end 116.15 80.16) (width 0.25) (layer "B.Cu") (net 12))
 (segment (start 87.01 80.19) (end 89.55 80.19) (width 0.25) (layer "B.Cu") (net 12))
 (segment (start 119.5 69.930914) (end 119.5 76.81) (width 0.25) (layer "B.Cu") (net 12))
 (segment (start 113.61 80.16) (end 116.15 80.16) (width 0.25) (layer "B.Cu") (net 12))
 (segment (start 89.55 78.85) (end 91.65 76.75) (width 0.25) (layer "B.Cu") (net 12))
 (segment (start 89.55 80.19) (end 89.55 78.85) (width 0.25) (layer "B.Cu") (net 12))
 (segment (start 101.525 60.24) (end 101.525 63.365) (width 0.25) (layer "B.Cu") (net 12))
 (segment (start 101.525 63.365) (end 101.75 63.59) (width 0.25) (layer "B.Cu") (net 12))
 (segment (start 88.387289 86.432711) (end 88.387289 62.712711) (width 0.25) (layer "F.Cu") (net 13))
 (segment (start 89.3 61.8) (end 92.345 61.8) (width 0.25) (layer "F.Cu") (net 13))
 (segment (start 87.01 87.81) (end 88.387289 86.432711) (width 0.25) (layer "F.Cu") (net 13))
 (segment (start 88.387289 62.712711) (end 89.3 61.8) (width 0.25) (layer "F.Cu") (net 13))
 (segment (start 92.345 61.8) (end 93.905 60.24) (width 0.25) (layer "F.Cu") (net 13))
 (segment (start 111.07 87.78) (end 106.402231 83.112231) (width 0.25) (layer "B.Cu") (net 13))
 (segment (start 106.402231 72.737231) (end 93.905 60.24) (width 0.25) (layer "B.Cu") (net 13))
 (segment (start 106.402231 83.112231) (end 106.402231 72.737231) (width 0.25) (layer "B.Cu") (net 13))
 (segment (start 89.55 87.81) (end 90.712711 86.647289) (width 0.25) (layer "F.Cu") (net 14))
 (segment (start 90.712711 73.746167) (end 96.445 68.013878) (width 0.25) (layer "F.Cu") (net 14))
 (segment (start 90.712711 86.647289) (end 90.712711 73.746167) (width 0.25) (layer "F.Cu") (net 14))
 (segment (start 96.445 68.013878) (end 96.445 60.24) (width 0.25) (layer "F.Cu") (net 14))
 (segment (start 109.907289 75.606571) (end 96.445 62.144282) (width 0.25) (layer "B.Cu") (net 14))
 (segment (start 113.61 87.78) (end 109.907289 84.077289) (width 0.25) (layer "B.Cu") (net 14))
 (segment (start 96.445 62.144282) (end 96.445 60.24) (width 0.25) (layer "B.Cu") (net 14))
 (segment (start 109.907289 84.077289) (end 109.907289 75.606571) (width 0.25) (layer "B.Cu") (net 14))
 (segment (start 93.45 71.644596) (end 98.985 66.109596) (width 0.25) (layer "F.Cu") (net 15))
 (segment (start 93.45 80.474323) (end 93.45 71.644596) (width 0.25) (layer "F.Cu") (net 15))
 (segment (start 92.09 87.81) (end 92.09 81.834323) (width 0.25) (layer "F.Cu") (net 15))
 (segment (start 98.985 66.109596) (end 98.985 60.24) (width 0.25) (layer "F.Cu") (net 15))
 (segment (start 92.09 81.834323) (end 93.45 80.474323) (width 0.25) (layer "F.Cu") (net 15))
 (segment (start 116.15 87.78) (end 112.232711 83.862711) (width 0.25) (layer "B.Cu") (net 15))
 (segment (start 112.232711 75.532711) (end 98.985 62.285) (width 0.25) (layer "B.Cu") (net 15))
 (segment (start 98.985 62.285) (end 98.985 60.24) (width 0.25) (layer "B.Cu") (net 15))
 (segment (start 112.232711 83.862711) (end 112.232711 75.532711) (width 0.25) (layer "B.Cu") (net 15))
 (segment (start 105.952711 57.047711) (end 101.525 52.62) (width 0.25) (layer "F.Cu") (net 18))
 (segment (start 104.79 87.81) (end 107 85.6) (width 0.25) (layer "F.Cu") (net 18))
 (segment (start 87.383511 123.807403) (end 121.686489 123.807403) (width 0.25) (layer "F.Cu") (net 18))
 (segment (start 101.525 52.62) (end 116.810914 52.62) (width 0.25) (layer "F.Cu") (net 18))
 (segment (start 121.686489 123.807403) (end 122.76 124.880914) (width 0.25) (layer "F.Cu") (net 18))
 (segment (start 104.79 87.81) (end 105.952711 86.647289) (width 0.25) (layer "F.Cu") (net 18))
 (segment (start 107 85.6) (end 120.35 85.6) (width 0.25) (layer "F.Cu") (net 18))
 (segment (start 116.810914 52.62) (end 119.5 49.930914) (width 0.25) (layer "F.Cu") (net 18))
 (segment (start 105.952711 86.647289) (end 105.952711 57.047711) (width 0.25) (layer "F.Cu") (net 18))
 (segment (start 86.31 124.880914) (end 87.383511 123.807403) (width 0.25) (layer "F.Cu") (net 18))
 (via (at 120.35 85.6) (size 0.8) (drill 0.4) (layers "F.Cu" "B.Cu") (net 18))
 (segment (start 126.67 85.6) (end 128.85 87.78) (width 0.25) (layer "B.Cu") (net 18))
 (segment (start 120.35 85.6) (end 126.67 85.6) (width 0.25) (layer "B.Cu") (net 18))
 (segment (start 128.85 118.790914) (end 128.85 87.78) (width 0.25) (layer "B.Cu") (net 18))
 (segment (start 122.76 124.880914) (end 128.85 118.790914) (width 0.25) (layer "B.Cu") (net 18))
 (segment (start 91.365 63.955) (end 91.4 63.99) (width 0.25) (layer "B.Cu") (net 26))
 (segment (start 91.365 60.24) (end 91.365 63.955) (width 0.25) (layer "B.Cu") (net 26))
 (segment (start 91.011122 65.05) (end 88.825 62.863878) (width 0.25) (layer "B.Cu") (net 10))
 (segment (start 88.825 62.863878) (end 88.825 60.24) (width 0.25) (layer "B.Cu") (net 10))
 (segment (start 97.038878 65.05) (end 91.011122 65.05) (width 0.25) (layer "B.Cu") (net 10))
 (segment (start 102.774511 77.125489) (end 102.774511 70.785633) (width 0.25) (layer "B.Cu") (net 10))
 (segment (start 99.71 80.19) (end 102.774511 77.125489) (width 0.25) (layer "B.Cu") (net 10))
 (segment (start 102.774511 70.785633) (end 97.038878 65.05) (width 0.25) (layer "B.Cu") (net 10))
 (segment (start 86.285 63.805) (end 86.25 63.84) (width 0.25) (layer "B.Cu") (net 25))
 (segment (start 86.285 60.24) (end 86.285 63.805) (width 0.25) (layer "B.Cu") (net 25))
 (segment (start 85.75 51.05) (end 87.255 51.05) (width 0.25) (layer "F.Cu") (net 23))
 (segment (start 84.6 52.2) (end 85.75 51.05) (width 0.25) (layer "F.Cu") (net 23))
 (segment (start 87.255 51.05) (end 88.825 52.62) (width 0.25) (layer "F.Cu") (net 23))
 (segment (start 84.6 127.520914) (end 84.6 52.2) (width 0.25) (layer "F.Cu") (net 23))
 (segment (start 86.46 129.380914) (end 84.6 127.520914) (width 0.25) (layer "F.Cu") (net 23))
 (segment (start 121.836489 130.454425) (end 85.254425 130.454425) (width 0.25) (layer "F.Cu") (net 22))
 (segment (start 83.85 129.05) (end 83.85 52.2) (width 0.25) (layer "F.Cu") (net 22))
 (segment (start 83.85 52.2) (end 85.44952 50.60048) (width 0.25) (layer "F.Cu") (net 22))
 (segment (start 85.44952 50.60048) (end 89.34548 50.60048) (width 0.25) (layer "F.Cu") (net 22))
 (segment (start 122.91 129.380914) (end 121.836489 130.454425) (width 0.25) (layer "F.Cu") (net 22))
 (segment (start 85.254425 130.454425) (end 83.85 129.05) (width 0.25) (layer "F.Cu") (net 22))
 (segment (start 89.34548 50.60048) (end 91.365 52.62) (width 0.25) (layer "F.Cu") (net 22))
 (segment (start 92.81 124.880914) (end 93.883511 125.954425) (width 0.25) (layer "F.Cu") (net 28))
 (segment (start 93.883511 125.954425) (end 128.186489 125.954425) (width 0.25) (layer "F.Cu") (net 28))
 (segment (start 128.186489 125.954425) (end 129.26 124.880914) (width 0.25) (layer "F.Cu") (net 28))
 (segment (start 92.81 124.880914) (end 90.927289 122.998203) (width 0.25) (layer "B.Cu") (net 28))
 (segment (start 90.927289 122.998203) (end 90.927289 79.708388) (width 0.25) (layer "B.Cu") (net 28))
 (segment (start 99.425677 71.21) (end 101.75 71.21) (width 0.25) (layer "B.Cu") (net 28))
 (segment (start 90.927289 79.708388) (end 99.425677 71.21) (width 0.25) (layer "B.Cu") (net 28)))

